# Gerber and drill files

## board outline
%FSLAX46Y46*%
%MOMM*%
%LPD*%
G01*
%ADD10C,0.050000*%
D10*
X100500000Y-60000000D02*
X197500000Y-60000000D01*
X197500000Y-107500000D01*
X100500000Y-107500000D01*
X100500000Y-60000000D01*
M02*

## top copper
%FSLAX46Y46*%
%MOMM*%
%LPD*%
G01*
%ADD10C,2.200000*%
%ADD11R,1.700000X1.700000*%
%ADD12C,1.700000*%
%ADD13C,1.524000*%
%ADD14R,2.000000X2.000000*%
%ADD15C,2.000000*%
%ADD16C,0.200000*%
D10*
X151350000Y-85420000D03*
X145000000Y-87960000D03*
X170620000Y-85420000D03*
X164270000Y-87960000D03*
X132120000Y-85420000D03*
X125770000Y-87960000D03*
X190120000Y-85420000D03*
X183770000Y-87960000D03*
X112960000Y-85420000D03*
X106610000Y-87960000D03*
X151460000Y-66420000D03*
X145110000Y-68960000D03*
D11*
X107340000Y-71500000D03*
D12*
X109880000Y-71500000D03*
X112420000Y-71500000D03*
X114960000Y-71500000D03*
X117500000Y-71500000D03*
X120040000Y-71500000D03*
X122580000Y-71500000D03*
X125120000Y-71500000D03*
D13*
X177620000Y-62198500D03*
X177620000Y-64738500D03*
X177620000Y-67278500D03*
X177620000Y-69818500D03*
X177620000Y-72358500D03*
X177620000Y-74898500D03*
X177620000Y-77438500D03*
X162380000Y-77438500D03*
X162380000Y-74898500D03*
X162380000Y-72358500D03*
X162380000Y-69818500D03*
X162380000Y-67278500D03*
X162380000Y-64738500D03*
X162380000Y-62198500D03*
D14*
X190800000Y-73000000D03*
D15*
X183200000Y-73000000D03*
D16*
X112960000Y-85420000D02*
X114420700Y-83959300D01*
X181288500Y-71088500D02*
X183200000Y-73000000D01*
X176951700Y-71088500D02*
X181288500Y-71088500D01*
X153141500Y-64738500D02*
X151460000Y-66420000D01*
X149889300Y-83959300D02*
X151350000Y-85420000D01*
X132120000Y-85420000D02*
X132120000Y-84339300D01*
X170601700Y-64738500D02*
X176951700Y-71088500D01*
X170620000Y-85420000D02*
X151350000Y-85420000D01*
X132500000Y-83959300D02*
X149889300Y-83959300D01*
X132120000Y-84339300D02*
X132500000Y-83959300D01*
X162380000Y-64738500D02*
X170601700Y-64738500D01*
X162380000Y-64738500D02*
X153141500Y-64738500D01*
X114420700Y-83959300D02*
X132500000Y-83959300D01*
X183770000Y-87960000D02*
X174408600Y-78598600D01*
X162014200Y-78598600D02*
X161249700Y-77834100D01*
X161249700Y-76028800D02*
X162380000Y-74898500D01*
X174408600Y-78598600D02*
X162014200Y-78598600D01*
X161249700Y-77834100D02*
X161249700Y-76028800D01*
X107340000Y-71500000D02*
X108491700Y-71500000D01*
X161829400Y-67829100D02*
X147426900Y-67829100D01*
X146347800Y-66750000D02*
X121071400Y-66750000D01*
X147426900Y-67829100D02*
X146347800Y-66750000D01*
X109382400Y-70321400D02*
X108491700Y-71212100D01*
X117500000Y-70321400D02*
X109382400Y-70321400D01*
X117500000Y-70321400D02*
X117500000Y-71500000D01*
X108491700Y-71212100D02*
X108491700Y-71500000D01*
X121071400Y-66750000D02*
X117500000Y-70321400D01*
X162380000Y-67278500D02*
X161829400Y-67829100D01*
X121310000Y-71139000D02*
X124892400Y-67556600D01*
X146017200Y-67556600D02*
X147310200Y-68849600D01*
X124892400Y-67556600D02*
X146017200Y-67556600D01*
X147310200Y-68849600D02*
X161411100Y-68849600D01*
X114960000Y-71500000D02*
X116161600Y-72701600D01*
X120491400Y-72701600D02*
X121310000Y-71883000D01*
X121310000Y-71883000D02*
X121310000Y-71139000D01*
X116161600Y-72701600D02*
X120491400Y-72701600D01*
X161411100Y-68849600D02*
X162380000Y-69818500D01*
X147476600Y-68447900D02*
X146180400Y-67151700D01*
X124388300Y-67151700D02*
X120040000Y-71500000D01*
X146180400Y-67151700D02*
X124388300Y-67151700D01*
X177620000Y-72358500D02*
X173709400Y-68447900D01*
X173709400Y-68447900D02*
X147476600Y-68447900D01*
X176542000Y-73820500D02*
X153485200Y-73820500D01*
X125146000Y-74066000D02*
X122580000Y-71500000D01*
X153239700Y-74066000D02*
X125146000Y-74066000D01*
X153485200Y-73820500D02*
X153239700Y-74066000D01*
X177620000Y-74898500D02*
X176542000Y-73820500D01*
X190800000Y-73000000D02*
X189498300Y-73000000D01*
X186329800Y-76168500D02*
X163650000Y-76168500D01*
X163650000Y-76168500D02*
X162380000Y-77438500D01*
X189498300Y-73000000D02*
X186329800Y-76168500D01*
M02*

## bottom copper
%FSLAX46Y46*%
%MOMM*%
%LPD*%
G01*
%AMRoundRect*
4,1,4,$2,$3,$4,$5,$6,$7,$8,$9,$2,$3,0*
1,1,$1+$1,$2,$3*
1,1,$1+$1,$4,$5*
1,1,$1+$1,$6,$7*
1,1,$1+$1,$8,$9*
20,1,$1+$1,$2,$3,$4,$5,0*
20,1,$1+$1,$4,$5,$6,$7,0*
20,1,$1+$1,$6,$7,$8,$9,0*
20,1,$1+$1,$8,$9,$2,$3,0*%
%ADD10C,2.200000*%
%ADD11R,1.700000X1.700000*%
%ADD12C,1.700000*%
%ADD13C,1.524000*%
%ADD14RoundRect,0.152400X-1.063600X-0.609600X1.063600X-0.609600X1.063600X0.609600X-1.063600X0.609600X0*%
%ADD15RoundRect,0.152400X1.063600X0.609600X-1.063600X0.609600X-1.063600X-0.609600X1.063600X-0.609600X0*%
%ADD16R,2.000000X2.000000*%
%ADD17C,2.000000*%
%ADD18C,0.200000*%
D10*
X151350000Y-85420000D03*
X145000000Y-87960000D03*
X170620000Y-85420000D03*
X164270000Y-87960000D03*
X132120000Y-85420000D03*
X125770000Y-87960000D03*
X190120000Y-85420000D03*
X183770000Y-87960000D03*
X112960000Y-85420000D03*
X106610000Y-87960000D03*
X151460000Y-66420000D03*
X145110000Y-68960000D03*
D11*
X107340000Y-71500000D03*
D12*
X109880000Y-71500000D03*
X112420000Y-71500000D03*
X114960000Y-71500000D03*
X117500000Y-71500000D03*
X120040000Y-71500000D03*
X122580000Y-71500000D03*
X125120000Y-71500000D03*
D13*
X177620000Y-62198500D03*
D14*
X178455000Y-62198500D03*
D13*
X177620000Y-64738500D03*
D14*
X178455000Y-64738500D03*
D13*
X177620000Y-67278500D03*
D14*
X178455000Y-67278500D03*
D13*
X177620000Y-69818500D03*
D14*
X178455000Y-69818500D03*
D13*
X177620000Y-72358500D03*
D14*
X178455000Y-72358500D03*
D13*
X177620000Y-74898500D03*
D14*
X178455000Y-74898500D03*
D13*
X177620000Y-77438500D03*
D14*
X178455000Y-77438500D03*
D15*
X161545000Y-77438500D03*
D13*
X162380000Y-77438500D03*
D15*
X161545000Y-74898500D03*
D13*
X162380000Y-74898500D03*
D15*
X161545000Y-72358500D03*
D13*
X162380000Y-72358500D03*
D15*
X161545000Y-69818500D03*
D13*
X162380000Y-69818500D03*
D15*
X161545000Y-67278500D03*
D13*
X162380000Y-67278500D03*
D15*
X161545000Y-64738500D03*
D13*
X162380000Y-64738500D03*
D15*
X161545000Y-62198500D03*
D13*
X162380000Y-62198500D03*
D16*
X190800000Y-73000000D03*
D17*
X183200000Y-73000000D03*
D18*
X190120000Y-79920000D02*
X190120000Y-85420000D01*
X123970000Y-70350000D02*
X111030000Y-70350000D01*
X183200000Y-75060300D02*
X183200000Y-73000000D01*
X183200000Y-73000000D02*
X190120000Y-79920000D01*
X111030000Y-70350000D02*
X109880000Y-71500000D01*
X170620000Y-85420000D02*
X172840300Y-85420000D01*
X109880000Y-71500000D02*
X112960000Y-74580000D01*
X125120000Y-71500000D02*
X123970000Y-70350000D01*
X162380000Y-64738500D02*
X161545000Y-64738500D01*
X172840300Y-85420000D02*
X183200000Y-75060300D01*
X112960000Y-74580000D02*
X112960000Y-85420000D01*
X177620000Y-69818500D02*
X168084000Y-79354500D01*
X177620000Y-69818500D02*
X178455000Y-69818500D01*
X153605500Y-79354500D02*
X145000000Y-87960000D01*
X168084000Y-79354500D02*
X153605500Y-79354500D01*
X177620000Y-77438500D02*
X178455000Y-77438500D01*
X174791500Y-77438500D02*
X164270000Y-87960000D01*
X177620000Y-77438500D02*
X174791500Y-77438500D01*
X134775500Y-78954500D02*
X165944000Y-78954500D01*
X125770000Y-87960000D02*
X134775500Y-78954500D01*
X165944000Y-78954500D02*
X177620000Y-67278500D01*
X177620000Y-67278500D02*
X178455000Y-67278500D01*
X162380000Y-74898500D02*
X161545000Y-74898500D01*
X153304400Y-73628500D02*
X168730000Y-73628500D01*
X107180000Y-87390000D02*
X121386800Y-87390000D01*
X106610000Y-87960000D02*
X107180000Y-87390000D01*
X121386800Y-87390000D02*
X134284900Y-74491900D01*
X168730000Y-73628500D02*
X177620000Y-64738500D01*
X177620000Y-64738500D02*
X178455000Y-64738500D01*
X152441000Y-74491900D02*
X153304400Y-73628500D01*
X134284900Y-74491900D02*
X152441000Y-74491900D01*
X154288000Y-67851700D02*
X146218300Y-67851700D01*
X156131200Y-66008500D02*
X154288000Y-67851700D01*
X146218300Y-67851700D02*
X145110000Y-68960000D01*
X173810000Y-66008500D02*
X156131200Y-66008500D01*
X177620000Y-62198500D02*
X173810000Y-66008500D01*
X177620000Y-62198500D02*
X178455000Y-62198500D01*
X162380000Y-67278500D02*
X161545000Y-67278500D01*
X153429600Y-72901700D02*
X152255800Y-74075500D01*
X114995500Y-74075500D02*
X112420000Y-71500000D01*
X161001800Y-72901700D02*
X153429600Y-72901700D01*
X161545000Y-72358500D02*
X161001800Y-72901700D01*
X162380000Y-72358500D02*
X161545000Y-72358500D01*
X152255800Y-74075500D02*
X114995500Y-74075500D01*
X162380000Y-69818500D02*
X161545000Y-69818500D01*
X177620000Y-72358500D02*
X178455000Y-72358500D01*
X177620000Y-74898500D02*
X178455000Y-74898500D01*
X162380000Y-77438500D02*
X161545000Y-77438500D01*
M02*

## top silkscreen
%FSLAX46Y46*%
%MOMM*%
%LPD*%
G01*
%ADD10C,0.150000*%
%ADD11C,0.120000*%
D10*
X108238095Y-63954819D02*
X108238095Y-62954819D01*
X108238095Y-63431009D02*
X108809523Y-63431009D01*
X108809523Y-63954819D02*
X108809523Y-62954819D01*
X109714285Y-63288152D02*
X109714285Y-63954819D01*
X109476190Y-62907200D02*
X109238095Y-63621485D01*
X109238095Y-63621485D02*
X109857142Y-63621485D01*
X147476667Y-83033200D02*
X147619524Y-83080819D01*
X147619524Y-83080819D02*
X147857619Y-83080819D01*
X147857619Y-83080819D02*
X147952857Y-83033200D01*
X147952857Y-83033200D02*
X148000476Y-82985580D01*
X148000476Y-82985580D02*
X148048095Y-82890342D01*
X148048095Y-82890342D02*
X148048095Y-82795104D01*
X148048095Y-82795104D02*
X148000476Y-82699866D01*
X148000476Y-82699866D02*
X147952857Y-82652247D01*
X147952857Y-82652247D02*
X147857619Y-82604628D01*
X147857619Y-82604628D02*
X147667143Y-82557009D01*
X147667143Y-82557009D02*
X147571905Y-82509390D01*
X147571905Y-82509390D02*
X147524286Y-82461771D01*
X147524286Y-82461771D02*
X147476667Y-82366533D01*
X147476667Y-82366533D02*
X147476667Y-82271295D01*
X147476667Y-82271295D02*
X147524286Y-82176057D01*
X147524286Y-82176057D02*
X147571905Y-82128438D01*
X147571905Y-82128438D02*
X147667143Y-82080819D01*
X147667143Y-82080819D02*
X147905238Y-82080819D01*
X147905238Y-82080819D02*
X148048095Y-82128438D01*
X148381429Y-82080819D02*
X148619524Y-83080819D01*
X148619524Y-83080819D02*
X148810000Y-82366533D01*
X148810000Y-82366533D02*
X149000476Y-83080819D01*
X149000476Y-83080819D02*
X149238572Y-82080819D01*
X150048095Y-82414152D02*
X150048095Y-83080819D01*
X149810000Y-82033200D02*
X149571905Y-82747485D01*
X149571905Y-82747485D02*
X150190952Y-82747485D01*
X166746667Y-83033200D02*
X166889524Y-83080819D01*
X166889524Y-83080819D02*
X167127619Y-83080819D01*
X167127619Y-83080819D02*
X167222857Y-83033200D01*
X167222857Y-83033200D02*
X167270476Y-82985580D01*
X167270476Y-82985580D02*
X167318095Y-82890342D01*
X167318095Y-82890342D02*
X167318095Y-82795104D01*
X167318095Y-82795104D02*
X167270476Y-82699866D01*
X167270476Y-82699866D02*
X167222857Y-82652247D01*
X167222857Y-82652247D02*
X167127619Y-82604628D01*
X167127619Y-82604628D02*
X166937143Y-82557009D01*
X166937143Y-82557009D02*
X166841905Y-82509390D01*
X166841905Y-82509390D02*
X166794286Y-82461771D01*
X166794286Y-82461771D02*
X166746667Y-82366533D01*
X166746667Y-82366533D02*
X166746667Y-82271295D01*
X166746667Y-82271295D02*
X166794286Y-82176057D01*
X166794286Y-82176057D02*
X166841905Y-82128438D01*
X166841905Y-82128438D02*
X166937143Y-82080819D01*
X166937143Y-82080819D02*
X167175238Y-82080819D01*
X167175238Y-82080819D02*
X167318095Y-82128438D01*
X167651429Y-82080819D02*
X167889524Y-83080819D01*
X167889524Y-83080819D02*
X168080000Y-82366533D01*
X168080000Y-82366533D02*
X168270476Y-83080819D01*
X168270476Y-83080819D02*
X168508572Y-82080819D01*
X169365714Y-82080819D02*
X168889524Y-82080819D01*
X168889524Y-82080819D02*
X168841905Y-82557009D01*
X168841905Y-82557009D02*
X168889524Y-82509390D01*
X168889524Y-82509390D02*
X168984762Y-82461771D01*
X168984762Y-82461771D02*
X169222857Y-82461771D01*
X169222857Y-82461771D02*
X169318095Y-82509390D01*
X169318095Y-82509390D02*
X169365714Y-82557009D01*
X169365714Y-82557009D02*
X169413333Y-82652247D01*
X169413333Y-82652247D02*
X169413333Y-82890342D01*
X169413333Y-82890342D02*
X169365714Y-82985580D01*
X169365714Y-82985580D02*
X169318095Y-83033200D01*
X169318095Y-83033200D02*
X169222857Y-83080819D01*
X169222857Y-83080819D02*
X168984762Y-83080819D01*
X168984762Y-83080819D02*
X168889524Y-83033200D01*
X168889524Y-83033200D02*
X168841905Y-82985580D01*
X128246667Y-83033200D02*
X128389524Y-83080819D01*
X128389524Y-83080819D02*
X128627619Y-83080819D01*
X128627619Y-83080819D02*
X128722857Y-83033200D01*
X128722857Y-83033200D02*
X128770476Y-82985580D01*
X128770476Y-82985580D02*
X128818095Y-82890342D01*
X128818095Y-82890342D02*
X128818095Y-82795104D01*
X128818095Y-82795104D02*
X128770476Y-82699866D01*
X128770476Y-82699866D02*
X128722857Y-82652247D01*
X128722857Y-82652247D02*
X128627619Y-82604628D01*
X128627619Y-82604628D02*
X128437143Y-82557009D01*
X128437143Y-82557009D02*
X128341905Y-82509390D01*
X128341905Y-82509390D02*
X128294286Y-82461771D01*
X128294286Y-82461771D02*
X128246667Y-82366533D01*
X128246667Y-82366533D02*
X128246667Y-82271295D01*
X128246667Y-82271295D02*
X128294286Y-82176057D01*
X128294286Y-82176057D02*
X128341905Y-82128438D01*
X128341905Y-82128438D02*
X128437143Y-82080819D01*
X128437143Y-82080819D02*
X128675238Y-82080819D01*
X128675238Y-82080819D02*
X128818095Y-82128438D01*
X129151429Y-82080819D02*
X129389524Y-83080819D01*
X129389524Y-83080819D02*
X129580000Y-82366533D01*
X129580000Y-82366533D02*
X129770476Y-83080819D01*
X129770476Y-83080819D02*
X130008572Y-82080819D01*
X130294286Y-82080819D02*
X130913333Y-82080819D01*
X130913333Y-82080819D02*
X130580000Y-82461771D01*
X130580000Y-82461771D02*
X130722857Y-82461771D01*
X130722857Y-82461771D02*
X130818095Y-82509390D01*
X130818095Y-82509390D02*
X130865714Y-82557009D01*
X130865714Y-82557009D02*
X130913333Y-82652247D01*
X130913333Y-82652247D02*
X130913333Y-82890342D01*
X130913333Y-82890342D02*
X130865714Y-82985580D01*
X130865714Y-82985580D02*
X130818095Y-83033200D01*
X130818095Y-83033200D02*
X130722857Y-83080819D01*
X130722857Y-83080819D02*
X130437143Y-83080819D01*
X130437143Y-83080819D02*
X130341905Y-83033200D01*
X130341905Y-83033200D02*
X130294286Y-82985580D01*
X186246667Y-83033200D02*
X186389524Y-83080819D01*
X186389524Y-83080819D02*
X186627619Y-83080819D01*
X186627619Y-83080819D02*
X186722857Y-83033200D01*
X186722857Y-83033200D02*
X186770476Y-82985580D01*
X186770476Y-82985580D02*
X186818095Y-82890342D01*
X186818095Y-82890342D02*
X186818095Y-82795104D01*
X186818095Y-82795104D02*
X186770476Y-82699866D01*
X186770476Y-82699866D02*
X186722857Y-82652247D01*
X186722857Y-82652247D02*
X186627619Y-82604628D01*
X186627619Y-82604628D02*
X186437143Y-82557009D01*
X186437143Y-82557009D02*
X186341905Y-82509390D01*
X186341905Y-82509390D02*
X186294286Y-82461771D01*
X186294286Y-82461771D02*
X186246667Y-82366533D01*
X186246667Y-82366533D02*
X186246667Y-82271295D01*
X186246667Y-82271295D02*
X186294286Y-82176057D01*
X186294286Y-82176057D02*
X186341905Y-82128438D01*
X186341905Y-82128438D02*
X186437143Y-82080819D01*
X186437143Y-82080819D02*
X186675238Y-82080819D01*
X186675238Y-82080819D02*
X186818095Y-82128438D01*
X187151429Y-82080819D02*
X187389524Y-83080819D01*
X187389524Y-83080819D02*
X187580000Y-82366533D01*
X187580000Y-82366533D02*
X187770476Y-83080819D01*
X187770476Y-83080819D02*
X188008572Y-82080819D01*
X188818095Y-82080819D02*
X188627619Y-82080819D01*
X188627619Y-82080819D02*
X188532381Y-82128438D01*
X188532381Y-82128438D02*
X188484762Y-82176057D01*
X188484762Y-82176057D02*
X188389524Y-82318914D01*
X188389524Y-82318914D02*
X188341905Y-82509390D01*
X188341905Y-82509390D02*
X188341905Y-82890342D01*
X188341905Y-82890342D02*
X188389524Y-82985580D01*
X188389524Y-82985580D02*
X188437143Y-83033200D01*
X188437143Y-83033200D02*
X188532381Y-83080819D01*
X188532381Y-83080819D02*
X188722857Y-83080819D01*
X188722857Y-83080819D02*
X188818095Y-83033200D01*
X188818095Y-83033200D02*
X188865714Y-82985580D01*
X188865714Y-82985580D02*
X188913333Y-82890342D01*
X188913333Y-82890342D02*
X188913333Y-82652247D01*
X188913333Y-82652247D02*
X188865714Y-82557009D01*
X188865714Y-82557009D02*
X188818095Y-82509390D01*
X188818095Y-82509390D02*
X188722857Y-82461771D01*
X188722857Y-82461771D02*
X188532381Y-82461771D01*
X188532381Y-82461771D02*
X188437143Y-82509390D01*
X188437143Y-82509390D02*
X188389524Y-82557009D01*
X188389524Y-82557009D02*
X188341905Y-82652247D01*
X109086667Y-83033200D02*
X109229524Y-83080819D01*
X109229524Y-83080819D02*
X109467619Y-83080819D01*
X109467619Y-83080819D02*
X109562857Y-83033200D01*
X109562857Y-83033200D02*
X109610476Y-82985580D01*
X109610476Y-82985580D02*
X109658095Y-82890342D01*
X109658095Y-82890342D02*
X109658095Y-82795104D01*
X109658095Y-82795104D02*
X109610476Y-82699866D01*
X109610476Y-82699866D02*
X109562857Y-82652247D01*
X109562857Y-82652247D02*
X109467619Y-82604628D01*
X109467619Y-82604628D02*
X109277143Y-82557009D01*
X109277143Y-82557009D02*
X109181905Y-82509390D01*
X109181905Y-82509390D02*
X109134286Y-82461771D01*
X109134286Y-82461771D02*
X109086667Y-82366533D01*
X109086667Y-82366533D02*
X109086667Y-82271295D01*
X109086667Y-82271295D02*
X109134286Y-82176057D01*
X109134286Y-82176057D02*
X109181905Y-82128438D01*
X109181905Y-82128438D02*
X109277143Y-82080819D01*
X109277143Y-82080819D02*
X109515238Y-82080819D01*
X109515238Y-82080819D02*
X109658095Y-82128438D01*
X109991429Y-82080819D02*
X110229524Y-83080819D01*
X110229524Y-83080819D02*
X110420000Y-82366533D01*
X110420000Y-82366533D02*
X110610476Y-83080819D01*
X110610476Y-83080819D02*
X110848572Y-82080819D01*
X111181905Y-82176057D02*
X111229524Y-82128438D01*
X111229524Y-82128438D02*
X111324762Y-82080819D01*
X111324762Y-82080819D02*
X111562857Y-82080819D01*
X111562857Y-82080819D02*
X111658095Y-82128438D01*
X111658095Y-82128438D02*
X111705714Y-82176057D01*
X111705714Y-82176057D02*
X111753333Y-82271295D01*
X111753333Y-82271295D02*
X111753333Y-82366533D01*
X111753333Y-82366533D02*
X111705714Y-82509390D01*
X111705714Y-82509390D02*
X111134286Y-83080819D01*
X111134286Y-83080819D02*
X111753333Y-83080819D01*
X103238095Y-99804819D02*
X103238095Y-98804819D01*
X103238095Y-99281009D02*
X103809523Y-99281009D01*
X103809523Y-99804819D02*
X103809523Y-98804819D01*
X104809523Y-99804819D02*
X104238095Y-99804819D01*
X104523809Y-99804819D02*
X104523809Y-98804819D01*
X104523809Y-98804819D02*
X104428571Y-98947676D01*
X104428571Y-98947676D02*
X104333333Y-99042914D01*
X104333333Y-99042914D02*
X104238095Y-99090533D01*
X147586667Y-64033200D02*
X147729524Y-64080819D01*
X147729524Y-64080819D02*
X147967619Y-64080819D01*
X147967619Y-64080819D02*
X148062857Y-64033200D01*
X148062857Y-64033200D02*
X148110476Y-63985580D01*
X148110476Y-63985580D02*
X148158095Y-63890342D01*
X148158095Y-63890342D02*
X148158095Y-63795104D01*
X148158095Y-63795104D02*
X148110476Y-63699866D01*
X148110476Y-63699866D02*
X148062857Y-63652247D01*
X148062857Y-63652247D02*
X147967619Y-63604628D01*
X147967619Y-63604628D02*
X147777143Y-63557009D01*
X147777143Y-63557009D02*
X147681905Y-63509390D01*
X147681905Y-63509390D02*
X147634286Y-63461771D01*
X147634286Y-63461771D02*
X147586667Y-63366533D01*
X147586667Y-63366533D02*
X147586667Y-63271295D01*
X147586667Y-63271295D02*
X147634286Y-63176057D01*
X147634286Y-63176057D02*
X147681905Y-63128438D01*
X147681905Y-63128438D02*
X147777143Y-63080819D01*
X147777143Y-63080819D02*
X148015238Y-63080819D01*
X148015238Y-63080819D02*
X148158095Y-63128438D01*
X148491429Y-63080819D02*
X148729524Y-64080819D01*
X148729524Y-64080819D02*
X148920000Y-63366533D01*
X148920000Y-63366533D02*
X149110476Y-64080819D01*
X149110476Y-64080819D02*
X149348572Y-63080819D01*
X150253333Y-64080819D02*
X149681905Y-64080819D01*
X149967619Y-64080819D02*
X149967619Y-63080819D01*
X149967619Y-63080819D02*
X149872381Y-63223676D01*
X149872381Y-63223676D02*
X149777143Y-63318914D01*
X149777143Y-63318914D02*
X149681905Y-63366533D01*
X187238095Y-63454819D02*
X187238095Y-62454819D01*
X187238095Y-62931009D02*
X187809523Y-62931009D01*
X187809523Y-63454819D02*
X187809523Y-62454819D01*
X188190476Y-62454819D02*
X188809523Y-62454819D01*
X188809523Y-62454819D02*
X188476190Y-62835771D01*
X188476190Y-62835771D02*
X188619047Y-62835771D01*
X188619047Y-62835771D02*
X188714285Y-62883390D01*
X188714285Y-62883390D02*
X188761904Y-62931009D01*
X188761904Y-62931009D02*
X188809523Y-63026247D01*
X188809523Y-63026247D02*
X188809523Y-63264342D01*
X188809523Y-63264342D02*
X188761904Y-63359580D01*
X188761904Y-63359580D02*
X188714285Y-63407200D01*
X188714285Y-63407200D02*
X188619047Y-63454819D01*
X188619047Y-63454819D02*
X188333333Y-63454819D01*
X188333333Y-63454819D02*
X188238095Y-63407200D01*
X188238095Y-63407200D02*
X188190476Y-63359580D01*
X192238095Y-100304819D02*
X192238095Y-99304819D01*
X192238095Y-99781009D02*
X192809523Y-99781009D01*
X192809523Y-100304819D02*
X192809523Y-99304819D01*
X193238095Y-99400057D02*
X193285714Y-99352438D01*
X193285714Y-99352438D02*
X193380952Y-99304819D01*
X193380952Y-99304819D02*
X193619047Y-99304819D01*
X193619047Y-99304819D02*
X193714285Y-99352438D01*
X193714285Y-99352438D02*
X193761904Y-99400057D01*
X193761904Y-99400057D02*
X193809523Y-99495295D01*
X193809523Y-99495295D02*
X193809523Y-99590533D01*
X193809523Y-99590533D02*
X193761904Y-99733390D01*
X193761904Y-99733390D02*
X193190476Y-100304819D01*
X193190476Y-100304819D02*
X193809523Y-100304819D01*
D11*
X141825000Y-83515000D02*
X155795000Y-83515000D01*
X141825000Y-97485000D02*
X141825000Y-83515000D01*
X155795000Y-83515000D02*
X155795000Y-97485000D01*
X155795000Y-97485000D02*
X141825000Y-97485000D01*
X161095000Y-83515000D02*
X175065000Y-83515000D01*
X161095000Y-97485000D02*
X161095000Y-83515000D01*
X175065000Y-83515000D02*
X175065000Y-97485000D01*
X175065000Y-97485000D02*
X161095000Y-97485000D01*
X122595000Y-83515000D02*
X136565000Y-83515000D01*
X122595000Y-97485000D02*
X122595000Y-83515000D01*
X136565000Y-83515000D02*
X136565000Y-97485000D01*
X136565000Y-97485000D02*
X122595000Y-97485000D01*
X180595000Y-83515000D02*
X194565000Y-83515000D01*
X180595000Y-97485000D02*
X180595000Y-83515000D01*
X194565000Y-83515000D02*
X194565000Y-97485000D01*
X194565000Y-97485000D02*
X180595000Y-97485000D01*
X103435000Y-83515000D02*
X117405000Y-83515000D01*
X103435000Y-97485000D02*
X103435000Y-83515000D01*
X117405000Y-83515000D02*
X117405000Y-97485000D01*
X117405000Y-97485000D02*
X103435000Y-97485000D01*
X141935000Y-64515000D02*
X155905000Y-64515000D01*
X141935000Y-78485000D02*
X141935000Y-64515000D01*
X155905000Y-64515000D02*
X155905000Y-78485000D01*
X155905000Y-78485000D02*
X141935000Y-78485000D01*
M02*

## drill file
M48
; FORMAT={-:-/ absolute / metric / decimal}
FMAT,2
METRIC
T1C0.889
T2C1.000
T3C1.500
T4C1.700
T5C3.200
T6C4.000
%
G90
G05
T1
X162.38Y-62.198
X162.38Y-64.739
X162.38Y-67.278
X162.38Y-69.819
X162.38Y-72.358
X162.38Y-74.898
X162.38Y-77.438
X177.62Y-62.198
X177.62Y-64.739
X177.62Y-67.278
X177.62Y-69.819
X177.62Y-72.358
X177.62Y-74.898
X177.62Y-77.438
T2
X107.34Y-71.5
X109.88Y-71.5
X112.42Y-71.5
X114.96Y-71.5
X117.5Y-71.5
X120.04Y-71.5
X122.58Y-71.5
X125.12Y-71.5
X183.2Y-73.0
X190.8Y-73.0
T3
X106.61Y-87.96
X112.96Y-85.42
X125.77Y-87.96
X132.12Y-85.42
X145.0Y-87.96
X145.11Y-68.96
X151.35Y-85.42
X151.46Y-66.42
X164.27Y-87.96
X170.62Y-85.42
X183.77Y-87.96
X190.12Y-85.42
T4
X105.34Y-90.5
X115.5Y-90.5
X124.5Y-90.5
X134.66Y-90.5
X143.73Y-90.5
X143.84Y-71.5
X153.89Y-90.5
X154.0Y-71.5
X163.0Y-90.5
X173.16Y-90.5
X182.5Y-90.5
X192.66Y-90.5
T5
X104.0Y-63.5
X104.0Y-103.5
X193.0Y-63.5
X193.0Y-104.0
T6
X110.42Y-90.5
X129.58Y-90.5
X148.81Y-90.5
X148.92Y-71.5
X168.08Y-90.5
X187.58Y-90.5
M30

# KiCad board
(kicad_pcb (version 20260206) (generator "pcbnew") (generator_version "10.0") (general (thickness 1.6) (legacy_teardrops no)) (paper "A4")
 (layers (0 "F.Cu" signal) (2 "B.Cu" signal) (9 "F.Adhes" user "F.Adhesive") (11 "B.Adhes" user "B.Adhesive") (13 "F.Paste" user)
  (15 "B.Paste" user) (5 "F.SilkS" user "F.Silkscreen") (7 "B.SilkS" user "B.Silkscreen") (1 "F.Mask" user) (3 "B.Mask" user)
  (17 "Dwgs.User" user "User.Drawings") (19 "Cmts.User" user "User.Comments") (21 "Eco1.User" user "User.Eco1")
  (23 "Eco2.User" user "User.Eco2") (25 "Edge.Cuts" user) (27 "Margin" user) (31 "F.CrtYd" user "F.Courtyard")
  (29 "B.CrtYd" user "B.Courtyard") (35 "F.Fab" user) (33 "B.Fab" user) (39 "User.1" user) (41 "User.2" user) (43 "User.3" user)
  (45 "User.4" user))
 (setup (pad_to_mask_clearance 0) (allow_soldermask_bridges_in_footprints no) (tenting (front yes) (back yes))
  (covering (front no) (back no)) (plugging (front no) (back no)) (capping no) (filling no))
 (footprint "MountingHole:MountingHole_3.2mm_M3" (layer "F.Cu") (at 104 63.5)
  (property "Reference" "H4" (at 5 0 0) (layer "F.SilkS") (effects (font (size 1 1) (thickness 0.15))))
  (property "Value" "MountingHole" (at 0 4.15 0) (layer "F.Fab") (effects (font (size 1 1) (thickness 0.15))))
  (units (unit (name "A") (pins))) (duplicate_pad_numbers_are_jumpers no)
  (pad "" np_thru_hole circle (at 0 0) (size 3.2 3.2) (drill 3.2) (layers "*.Cu" "*.Mask")))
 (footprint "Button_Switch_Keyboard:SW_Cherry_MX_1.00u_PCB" (layer "F.Cu") (at 151.35 85.42)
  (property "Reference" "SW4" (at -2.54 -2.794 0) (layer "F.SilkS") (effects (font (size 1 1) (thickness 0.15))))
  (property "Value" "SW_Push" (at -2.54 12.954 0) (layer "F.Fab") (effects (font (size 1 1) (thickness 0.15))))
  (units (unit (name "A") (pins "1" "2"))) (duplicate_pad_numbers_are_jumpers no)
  (fp_line (start -9.525 -1.905) (end 4.445 -1.905) (stroke (width 0.12) (type solid)) (layer "F.SilkS"))
  (fp_line (start -9.525 12.065) (end -9.525 -1.905) (stroke (width 0.12) (type solid)) (layer "F.SilkS"))
  (fp_line (start 4.445 -1.905) (end 4.445 12.065) (stroke (width 0.12) (type solid)) (layer "F.SilkS"))
  (fp_line (start 4.445 12.065) (end -9.525 12.065) (stroke (width 0.12) (type solid)) (layer "F.SilkS"))
  (pad "" np_thru_hole circle (at -7.62 5.08) (size 1.7 1.7) (drill 1.7) (layers "*.Cu" "*.Mask"))
  (pad "" np_thru_hole circle (at -2.54 5.08) (size 4 4) (drill 4) (layers "*.Cu" "*.Mask"))
  (pad "" np_thru_hole circle (at 2.54 5.08) (size 1.7 1.7) (drill 1.7) (layers "*.Cu" "*.Mask"))
  (pad "1" thru_hole circle (at 0 0) (size 2.2 2.2) (drill 1.5) (layers "*.Cu" "*.Mask") (remove_unused_layers no) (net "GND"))
  (pad "2" thru_hole circle (at -6.35 2.54) (size 2.2 2.2) (drill 1.5) (layers "*.Cu" "*.Mask") (remove_unused_layers no)
   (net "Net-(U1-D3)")))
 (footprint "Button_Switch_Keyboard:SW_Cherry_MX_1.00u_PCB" (layer "F.Cu") (at 170.62 85.42)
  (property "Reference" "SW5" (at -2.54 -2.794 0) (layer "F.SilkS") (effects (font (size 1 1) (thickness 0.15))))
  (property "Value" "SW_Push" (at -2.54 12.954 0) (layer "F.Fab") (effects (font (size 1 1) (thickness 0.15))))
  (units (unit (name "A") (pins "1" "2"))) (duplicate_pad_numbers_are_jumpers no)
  (fp_line (start -9.525 -1.905) (end 4.445 -1.905) (stroke (width 0.12) (type solid)) (layer "F.SilkS"))
  (fp_line (start -9.525 12.065) (end -9.525 -1.905) (stroke (width 0.12) (type solid)) (layer "F.SilkS"))
  (fp_line (start 4.445 -1.905) (end 4.445 12.065) (stroke (width 0.12) (type solid)) (layer "F.SilkS"))
  (fp_line (start 4.445 12.065) (end -9.525 12.065) (stroke (width 0.12) (type solid)) (layer "F.SilkS"))
  (pad "" np_thru_hole circle (at -7.62 5.08) (size 1.7 1.7) (drill 1.7) (layers "*.Cu" "*.Mask"))
  (pad "" np_thru_hole circle (at -2.54 5.08) (size 4 4) (drill 4) (layers "*.Cu" "*.Mask"))
  (pad "" np_thru_hole circle (at 2.54 5.08) (size 1.7 1.7) (drill 1.7) (layers "*.Cu" "*.Mask"))
  (pad "1" thru_hole circle (at 0 0) (size 2.2 2.2) (drill 1.5) (layers "*.Cu" "*.Mask") (remove_unused_layers no) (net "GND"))
  (pad "2" thru_hole circle (at -6.35 2.54) (size 2.2 2.2) (drill 1.5) (layers "*.Cu" "*.Mask") (remove_unused_layers no)
   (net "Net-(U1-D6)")))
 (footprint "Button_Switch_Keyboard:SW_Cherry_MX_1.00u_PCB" (layer "F.Cu") (at 132.12 85.42)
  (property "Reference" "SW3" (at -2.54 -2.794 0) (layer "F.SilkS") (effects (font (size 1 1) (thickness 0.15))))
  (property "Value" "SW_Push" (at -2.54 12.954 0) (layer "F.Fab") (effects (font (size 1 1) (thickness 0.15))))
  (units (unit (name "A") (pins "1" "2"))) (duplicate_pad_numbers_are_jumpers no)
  (fp_line (start -9.525 -1.905) (end 4.445 -1.905) (stroke (width 0.12) (type solid)) (layer "F.SilkS"))
  (fp_line (start -9.525 12.065) (end -9.525 -1.905) (stroke (width 0.12) (type solid)) (layer "F.SilkS"))
  (fp_line (start 4.445 -1.905) (end 4.445 12.065) (stroke (width 0.12) (type solid)) (layer "F.SilkS"))
  (fp_line (start 4.445 12.065) (end -9.525 12.065) (stroke (width 0.12) (type solid)) (layer "F.SilkS"))
  (pad "" np_thru_hole circle (at -7.62 5.08) (size 1.7 1.7) (drill 1.7) (layers "*.Cu" "*.Mask"))
  (pad "" np_thru_hole circle (at -2.54 5.08) (size 4 4) (drill 4) (layers "*.Cu" "*.Mask"))
  (pad "" np_thru_hole circle (at 2.54 5.08) (size 1.7 1.7) (drill 1.7) (layers "*.Cu" "*.Mask"))
  (pad "1" thru_hole circle (at 0 0) (size 2.2 2.2) (drill 1.5) (layers "*.Cu" "*.Mask") (remove_unused_layers no) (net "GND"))
  (pad "2" thru_hole circle (at -6.35 2.54) (size 2.2 2.2) (drill 1.5) (layers "*.Cu" "*.Mask") (remove_unused_layers no)
   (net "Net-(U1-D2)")))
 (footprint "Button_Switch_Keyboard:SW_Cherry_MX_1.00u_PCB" (layer "F.Cu") (at 190.12 85.42)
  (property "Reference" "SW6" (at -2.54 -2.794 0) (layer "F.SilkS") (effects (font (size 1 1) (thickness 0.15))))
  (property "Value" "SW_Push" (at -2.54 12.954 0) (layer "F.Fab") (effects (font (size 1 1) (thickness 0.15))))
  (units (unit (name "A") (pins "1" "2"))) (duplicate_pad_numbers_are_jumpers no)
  (fp_line (start -9.525 -1.905) (end 4.445 -1.905) (stroke (width 0.12) (type solid)) (layer "F.SilkS"))
  (fp_line (start -9.525 12.065) (end -9.525 -1.905) (stroke (width 0.12) (type solid)) (layer "F.SilkS"))
  (fp_line (start 4.445 -1.905) (end 4.445 12.065) (stroke (width 0.12) (type solid)) (layer "F.SilkS"))
  (fp_line (start 4.445 12.065) (end -9.525 12.065) (stroke (width 0.12) (type solid)) (layer "F.SilkS"))
  (pad "" np_thru_hole circle (at -7.62 5.08) (size 1.7 1.7) (drill 1.7) (layers "*.Cu" "*.Mask"))
  (pad "" np_thru_hole circle (at -2.54 5.08) (size 4 4) (drill 4) (layers "*.Cu" "*.Mask"))
  (pad "" np_thru_hole circle (at 2.54 5.08) (size 1.7 1.7) (drill 1.7) (layers "*.Cu" "*.Mask"))
  (pad "1" thru_hole circle (at 0 0) (size 2.2 2.2) (drill 1.5) (layers "*.Cu" "*.Mask") (remove_unused_layers no) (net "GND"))
  (pad "2" thru_hole circle (at -6.35 2.54) (size 2.2 2.2) (drill 1.5) (layers "*.Cu" "*.Mask") (remove_unused_layers no)
   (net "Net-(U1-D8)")))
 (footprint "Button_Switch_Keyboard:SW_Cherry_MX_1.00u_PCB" (layer "F.Cu") (at 112.96 85.42)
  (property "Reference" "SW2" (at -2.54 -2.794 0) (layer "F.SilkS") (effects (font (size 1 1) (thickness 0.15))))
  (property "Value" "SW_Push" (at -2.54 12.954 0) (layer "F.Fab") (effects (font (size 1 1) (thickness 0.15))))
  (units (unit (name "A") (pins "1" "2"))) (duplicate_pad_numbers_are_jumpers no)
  (fp_line (start -9.525 -1.905) (end 4.445 -1.905) (stroke (width 0.12) (type solid)) (layer "F.SilkS"))
  (fp_line (start -9.525 12.065) (end -9.525 -1.905) (stroke (width 0.12) (type solid)) (layer "F.SilkS"))
  (fp_line (start 4.445 -1.905) (end 4.445 12.065) (stroke (width 0.12) (type solid)) (layer "F.SilkS"))
  (fp_line (start 4.445 12.065) (end -9.525 12.065) (stroke (width 0.12) (type solid)) (layer "F.SilkS"))
  (pad "" np_thru_hole circle (at -7.62 5.08) (size 1.7 1.7) (drill 1.7) (layers "*.Cu" "*.Mask"))
  (pad "" np_thru_hole circle (at -2.54 5.08) (size 4 4) (drill 4) (layers "*.Cu" "*.Mask"))
  (pad "" np_thru_hole circle (at 2.54 5.08) (size 1.7 1.7) (drill 1.7) (layers "*.Cu" "*.Mask"))
  (pad "1" thru_hole circle (at 0 0) (size 2.2 2.2) (drill 1.5) (layers "*.Cu" "*.Mask") (remove_unused_layers no) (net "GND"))
  (pad "2" thru_hole circle (at -6.35 2.54) (size 2.2 2.2) (drill 1.5) (layers "*.Cu" "*.Mask") (remove_unused_layers no)
   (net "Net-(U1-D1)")))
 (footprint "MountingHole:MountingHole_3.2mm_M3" (layer "F.Cu") (at 104 103.5)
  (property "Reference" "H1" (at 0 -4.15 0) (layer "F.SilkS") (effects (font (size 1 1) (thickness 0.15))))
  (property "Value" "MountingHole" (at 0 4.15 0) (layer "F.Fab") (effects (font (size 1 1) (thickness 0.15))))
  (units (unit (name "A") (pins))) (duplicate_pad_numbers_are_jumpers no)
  (pad "" np_thru_hole circle (at 0 0) (size 3.2 3.2) (drill 3.2) (layers "*.Cu" "*.Mask")))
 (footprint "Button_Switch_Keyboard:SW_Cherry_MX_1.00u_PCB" (layer "F.Cu") (at 151.46 66.42)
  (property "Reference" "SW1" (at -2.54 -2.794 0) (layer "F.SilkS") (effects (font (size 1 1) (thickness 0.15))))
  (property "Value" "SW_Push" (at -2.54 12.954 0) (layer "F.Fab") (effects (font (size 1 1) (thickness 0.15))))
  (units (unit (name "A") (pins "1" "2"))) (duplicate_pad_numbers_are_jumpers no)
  (fp_line (start -9.525 -1.905) (end 4.445 -1.905) (stroke (width 0.12) (type solid)) (layer "F.SilkS"))
  (fp_line (start -9.525 12.065) (end -9.525 -1.905) (stroke (width 0.12) (type solid)) (layer "F.SilkS"))
  (fp_line (start 4.445 -1.905) (end 4.445 12.065) (stroke (width 0.12) (type solid)) (layer "F.SilkS"))
  (fp_line (start 4.445 12.065) (end -9.525 12.065) (stroke (width 0.12) (type solid)) (layer "F.SilkS"))
  (pad "" np_thru_hole circle (at -7.62 5.08) (size 1.7 1.7) (drill 1.7) (layers "*.Cu" "*.Mask"))
  (pad "" np_thru_hole circle (at -2.54 5.08) (size 4 4) (drill 4) (layers "*.Cu" "*.Mask"))
  (pad "" np_thru_hole circle (at 2.54 5.08) (size 1.7 1.7) (drill 1.7) (layers "*.Cu" "*.Mask"))
  (pad "1" thru_hole circle (at 0 0) (size 2.2 2.2) (drill 1.5) (layers "*.Cu" "*.Mask") (remove_unused_layers no) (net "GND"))
  (pad "2" thru_hole circle (at -6.35 2.54) (size 2.2 2.2) (drill 1.5) (layers "*.Cu" "*.Mask") (remove_unused_layers no)
   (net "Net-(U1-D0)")))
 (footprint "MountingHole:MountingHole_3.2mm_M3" (layer "F.Cu") (at 193 63.5)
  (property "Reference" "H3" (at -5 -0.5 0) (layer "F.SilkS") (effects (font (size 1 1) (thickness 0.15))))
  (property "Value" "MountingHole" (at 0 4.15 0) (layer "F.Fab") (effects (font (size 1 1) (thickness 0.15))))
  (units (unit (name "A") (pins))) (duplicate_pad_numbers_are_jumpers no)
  (pad "" np_thru_hole circle (at 0 0) (size 3.2 3.2) (drill 3.2) (layers "*.Cu" "*.Mask")))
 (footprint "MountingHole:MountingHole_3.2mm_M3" (layer "F.Cu") (at 193 104)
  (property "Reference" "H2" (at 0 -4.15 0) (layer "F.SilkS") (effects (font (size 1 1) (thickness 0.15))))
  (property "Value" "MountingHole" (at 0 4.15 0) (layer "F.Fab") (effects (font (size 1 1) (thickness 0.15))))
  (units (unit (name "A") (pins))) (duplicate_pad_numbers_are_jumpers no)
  (pad "" np_thru_hole circle (at 0 0) (size 3.2 3.2) (drill 3.2) (layers "*.Cu" "*.Mask")))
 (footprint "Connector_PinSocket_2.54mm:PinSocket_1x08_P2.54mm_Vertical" (layer "B.Cu") (at 107.34 71.5 -90)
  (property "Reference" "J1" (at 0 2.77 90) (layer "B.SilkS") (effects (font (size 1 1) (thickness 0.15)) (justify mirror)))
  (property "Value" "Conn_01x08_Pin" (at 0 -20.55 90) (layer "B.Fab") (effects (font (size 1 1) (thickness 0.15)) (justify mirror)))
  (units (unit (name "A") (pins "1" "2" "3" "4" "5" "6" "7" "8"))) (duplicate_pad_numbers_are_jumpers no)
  (pad "1" thru_hole rect (at 0 0 270) (size 1.7 1.7) (drill 1) (layers "*.Cu" "*.Mask") (remove_unused_layers no) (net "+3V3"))
  (pad "2" thru_hole circle (at 0 -2.54 270) (size 1.7 1.7) (drill 1) (layers "*.Cu" "*.Mask") (remove_unused_layers no) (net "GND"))
  (pad "3" thru_hole circle (at 0 -5.08 270) (size 1.7 1.7) (drill 1) (layers "*.Cu" "*.Mask") (remove_unused_layers no) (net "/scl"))
  (pad "4" thru_hole circle (at 0 -7.62 270) (size 1.7 1.7) (drill 1) (layers "*.Cu" "*.Mask") (remove_unused_layers no) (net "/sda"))
  (pad "5" thru_hole circle (at 0 -10.16 270) (size 1.7 1.7) (drill 1) (layers "*.Cu" "*.Mask") (remove_unused_layers no) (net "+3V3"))
  (pad "6" thru_hole circle (at 0 -12.7 270) (size 1.7 1.7) (drill 1) (layers "*.Cu" "*.Mask") (remove_unused_layers no) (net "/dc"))
  (pad "7" thru_hole circle (at 0 -15.24 270) (size 1.7 1.7) (drill 1) (layers "*.Cu" "*.Mask") (remove_unused_layers no) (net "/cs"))
  (pad "8" thru_hole circle (at 0 -17.78 270) (size 1.7 1.7) (drill 1) (layers "*.Cu" "*.Mask") (remove_unused_layers no) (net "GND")))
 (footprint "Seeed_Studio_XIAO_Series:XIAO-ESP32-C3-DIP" (layer "B.Cu") (at 170 69.8185 90)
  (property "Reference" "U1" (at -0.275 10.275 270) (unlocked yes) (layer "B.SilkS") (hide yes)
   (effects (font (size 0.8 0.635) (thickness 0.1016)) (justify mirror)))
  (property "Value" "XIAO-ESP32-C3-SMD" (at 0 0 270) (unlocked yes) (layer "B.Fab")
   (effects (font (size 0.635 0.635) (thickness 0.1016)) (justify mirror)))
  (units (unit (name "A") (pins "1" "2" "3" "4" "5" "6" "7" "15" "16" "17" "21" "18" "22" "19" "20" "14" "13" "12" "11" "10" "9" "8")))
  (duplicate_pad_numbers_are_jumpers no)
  (pad "1" thru_hole circle (at 7.62 7.62) (size 1.524 1.524) (drill 0.889) (layers "*.Cu" "*.Mask") (remove_unused_layers no)
   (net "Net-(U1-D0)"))
  (pad "1" smd roundrect (at 7.62 8.455) (size 2.432 1.524) (layers "B.Cu" "B.Mask") (roundrect_rratio 0.1) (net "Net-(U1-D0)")
   (thermal_bridge_angle 45))
  (pad "2" thru_hole circle (at 5.08 7.62) (size 1.524 1.524) (drill 0.889) (layers "*.Cu" "*.Mask") (remove_unused_layers no)
   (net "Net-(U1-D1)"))
  (pad "2" smd roundrect (at 5.08 8.455) (size 2.432 1.524) (layers "B.Cu" "B.Mask") (roundrect_rratio 0.1) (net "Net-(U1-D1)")
   (thermal_bridge_angle 45))
  (pad "3" thru_hole circle (at 2.54 7.62) (size 1.524 1.524) (drill 0.889) (layers "*.Cu" "*.Mask") (remove_unused_layers no)
   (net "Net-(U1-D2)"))
  (pad "3" smd roundrect (at 2.54 8.455) (size 2.432 1.524) (layers "B.Cu" "B.Mask") (roundrect_rratio 0.1) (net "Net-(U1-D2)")
   (thermal_bridge_angle 45))
  (pad "4" thru_hole circle (at 0 7.62) (size 1.524 1.524) (drill 0.889) (layers "*.Cu" "*.Mask") (remove_unused_layers no)
   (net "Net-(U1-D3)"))
  (pad "4" smd roundrect (at 0 8.455) (size 2.432 1.524) (layers "B.Cu" "B.Mask") (roundrect_rratio 0.1) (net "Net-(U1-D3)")
   (thermal_bridge_angle 45))
  (pad "5" thru_hole circle (at -2.54 7.62) (size 1.524 1.524) (drill 0.889) (layers "*.Cu" "*.Mask") (remove_unused_layers no) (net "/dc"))
  (pad "5" smd roundrect (at -2.54 8.455) (size 2.432 1.524) (layers "B.Cu" "B.Mask") (roundrect_rratio 0.1) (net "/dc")
   (thermal_bridge_angle 45))
  (pad "6" thru_hole circle (at -5.08 7.62) (size 1.524 1.524) (drill 0.889) (layers "*.Cu" "*.Mask") (remove_unused_layers no) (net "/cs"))
  (pad "6" smd roundrect (at -5.08 8.455) (size 2.432 1.524) (layers "B.Cu" "B.Mask") (roundrect_rratio 0.1) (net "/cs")
   (thermal_bridge_angle 45))
  (pad "7" thru_hole circle (at -7.62 7.62) (size 1.524 1.524) (drill 0.889) (layers "*.Cu" "*.Mask") (remove_unused_layers no)
   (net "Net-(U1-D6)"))
  (pad "7" smd roundrect (at -7.62 8.455) (size 2.432 1.524) (layers "B.Cu" "B.Mask") (roundrect_rratio 0.1) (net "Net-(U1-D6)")
   (thermal_bridge_angle 45))
  (pad "8" smd roundrect (at -7.62 -8.455 180) (size 2.432 1.524) (layers "B.Cu" "B.Mask") (roundrect_rratio 0.1) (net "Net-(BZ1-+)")
   (thermal_bridge_angle 45))
  (pad "8" thru_hole circle (at -7.62 -7.62 180) (size 1.524 1.524) (drill 0.889) (layers "*.Cu" "*.Mask") (remove_unused_layers no)
   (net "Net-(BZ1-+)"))
  (pad "9" smd roundrect (at -5.08 -8.455 180) (size 2.432 1.524) (layers "B.Cu" "B.Mask") (roundrect_rratio 0.1) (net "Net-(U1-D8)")
   (thermal_bridge_angle 45))
  (pad "9" thru_hole circle (at -5.08 -7.62 180) (size 1.524 1.524) (drill 0.889) (layers "*.Cu" "*.Mask") (remove_unused_layers no)
   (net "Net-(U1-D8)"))
  (pad "10" smd roundrect (at -2.54 -8.455 180) (size 2.432 1.524) (layers "B.Cu" "B.Mask") (roundrect_rratio 0.1) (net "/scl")
   (thermal_bridge_angle 45))
  (pad "10" thru_hole circle (at -2.54 -7.62 180) (size 1.524 1.524) (drill 0.889) (layers "*.Cu" "*.Mask") (remove_unused_layers no)
   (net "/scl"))
  (pad "11" smd roundrect (at 0 -8.455 180) (size 2.432 1.524) (layers "B.Cu" "B.Mask") (roundrect_rratio 0.1) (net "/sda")
   (thermal_bridge_angle 45))
  (pad "11" thru_hole circle (at 0 -7.62 180) (size 1.524 1.524) (drill 0.889) (layers "*.Cu" "*.Mask") (remove_unused_layers no)
   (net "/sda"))
  (pad "12" smd roundrect (at 2.54 -8.455 180) (size 2.432 1.524) (layers "B.Cu" "B.Mask") (roundrect_rratio 0.1) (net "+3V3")
   (thermal_bridge_angle 45))
  (pad "12" thru_hole circle (at 2.54 -7.62 180) (size 1.524 1.524) (drill 0.889) (layers "*.Cu" "*.Mask") (remove_unused_layers no)
   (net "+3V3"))
  (pad "13" smd roundrect (at 5.08 -8.455 180) (size 2.432 1.524) (layers "B.Cu" "B.Mask") (roundrect_rratio 0.1) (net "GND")
   (thermal_bridge_angle 45))
  (pad "13" thru_hole circle (at 5.08 -7.62 180) (size 1.524 1.524) (drill 0.889) (layers "*.Cu" "*.Mask") (remove_unused_layers no)
   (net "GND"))
  (pad "14" smd roundrect (at 7.62 -8.455 180) (size 2.432 1.524) (layers "B.Cu" "B.Mask") (roundrect_rratio 0.1)
   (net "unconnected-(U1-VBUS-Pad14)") (thermal_bridge_angle 45))
  (pad "14" thru_hole circle (at 7.62 -7.62 180) (size 1.524 1.524) (drill 0.889) (layers "*.Cu" "*.Mask") (remove_unused_layers no)
   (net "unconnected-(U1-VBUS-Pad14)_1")))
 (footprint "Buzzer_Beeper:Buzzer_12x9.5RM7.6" (layer "B.Cu") (at 190.8 73 180)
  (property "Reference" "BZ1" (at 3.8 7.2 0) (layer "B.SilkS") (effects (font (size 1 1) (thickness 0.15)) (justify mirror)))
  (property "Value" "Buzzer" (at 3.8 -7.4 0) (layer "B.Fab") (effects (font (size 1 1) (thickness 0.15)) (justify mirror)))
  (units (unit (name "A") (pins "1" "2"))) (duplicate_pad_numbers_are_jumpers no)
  (pad "1" thru_hole rect (at 0 0 180) (size 2 2) (drill 1) (layers "*.Cu" "*.Mask") (remove_unused_layers no) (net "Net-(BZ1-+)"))
  (pad "2" thru_hole circle (at 7.6 0 180) (size 2 2) (drill 1) (layers "*.Cu" "*.Mask") (remove_unused_layers no) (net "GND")))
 (gr_rect (start 100.5 60) (end 197.5 107.5) (stroke (width 0.05) (type default)) (fill no) (layer "Edge.Cuts"))
 (segment (start 112.96 85.42) (end 114.4207 83.9593) (width 0.2) (layer "F.Cu") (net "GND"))
 (segment (start 181.2885 71.0885) (end 183.2 73) (width 0.2) (layer "F.Cu") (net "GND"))
 (segment (start 176.9517 71.0885) (end 181.2885 71.0885) (width 0.2) (layer "F.Cu") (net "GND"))
 (segment (start 153.1415 64.7385) (end 151.46 66.42) (width 0.2) (layer "F.Cu") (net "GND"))
 (segment (start 149.8893 83.9593) (end 151.35 85.42) (width 0.2) (layer "F.Cu") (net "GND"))
 (segment (start 132.12 85.42) (end 132.12 84.3393) (width 0.2) (layer "F.Cu") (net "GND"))
 (segment (start 170.6017 64.7385) (end 176.9517 71.0885) (width 0.2) (layer "F.Cu") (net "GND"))
 (segment (start 170.62 85.42) (end 151.35 85.42) (width 0.2) (layer "F.Cu") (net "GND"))
 (segment (start 132.5 83.9593) (end 149.8893 83.9593) (width 0.2) (layer "F.Cu") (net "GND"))
 (segment (start 132.12 84.3393) (end 132.5 83.9593) (width 0.2) (layer "F.Cu") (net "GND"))
 (segment (start 162.38 64.7385) (end 170.6017 64.7385) (width 0.2) (layer "F.Cu") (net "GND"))
 (segment (start 162.38 64.7385) (end 153.1415 64.7385) (width 0.2) (layer "F.Cu") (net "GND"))
 (segment (start 114.4207 83.9593) (end 132.5 83.9593) (width 0.2) (layer "F.Cu") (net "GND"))
 (segment (start 190.12 79.92) (end 190.12 85.42) (width 0.2) (layer "B.Cu") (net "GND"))
 (segment (start 123.97 70.35) (end 111.03 70.35) (width 0.2) (layer "B.Cu") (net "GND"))
 (segment (start 183.2 75.0603) (end 183.2 73) (width 0.2) (layer "B.Cu") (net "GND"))
 (segment (start 183.2 73) (end 190.12 79.92) (width 0.2) (layer "B.Cu") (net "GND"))
 (segment (start 111.03 70.35) (end 109.88 71.5) (width 0.2) (layer "B.Cu") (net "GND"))
 (segment (start 170.62 85.42) (end 172.8403 85.42) (width 0.2) (layer "B.Cu") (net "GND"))
 (segment (start 109.88 71.5) (end 112.96 74.58) (width 0.2) (layer "B.Cu") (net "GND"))
 (segment (start 125.12 71.5) (end 123.97 70.35) (width 0.2) (layer "B.Cu") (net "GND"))
 (segment (start 162.38 64.7385) (end 161.545 64.7385) (width 0.2) (layer "B.Cu") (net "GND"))
 (segment (start 172.8403 85.42) (end 183.2 75.0603) (width 0.2) (layer "B.Cu") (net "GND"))
 (segment (start 112.96 74.58) (end 112.96 85.42) (width 0.2) (layer "B.Cu") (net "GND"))
 (segment (start 177.62 69.8185) (end 168.084 79.3545) (width 0.2) (layer "B.Cu") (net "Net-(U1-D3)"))
 (segment (start 177.62 69.8185) (end 178.455 69.8185) (width 0.2) (layer "B.Cu") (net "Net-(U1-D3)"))
 (segment (start 153.6055 79.3545) (end 145 87.96) (width 0.2) (layer "B.Cu") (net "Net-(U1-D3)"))
 (segment (start 168.084 79.3545) (end 153.6055 79.3545) (width 0.2) (layer "B.Cu") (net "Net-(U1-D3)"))
 (segment (start 177.62 77.4385) (end 178.455 77.4385) (width 0.2) (layer "B.Cu") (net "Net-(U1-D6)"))
 (segment (start 174.7915 77.4385) (end 164.27 87.96) (width 0.2) (layer "B.Cu") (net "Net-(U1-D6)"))
 (segment (start 177.62 77.4385) (end 174.7915 77.4385) (width 0.2) (layer "B.Cu") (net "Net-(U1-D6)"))
 (segment (start 134.7755 78.9545) (end 165.944 78.9545) (width 0.2) (layer "B.Cu") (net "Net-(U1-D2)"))
 (segment (start 125.77 87.96) (end 134.7755 78.9545) (width 0.2) (layer "B.Cu") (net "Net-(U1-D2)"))
 (segment (start 165.944 78.9545) (end 177.62 67.2785) (width 0.2) (layer "B.Cu") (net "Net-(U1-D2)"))
 (segment (start 177.62 67.2785) (end 178.455 67.2785) (width 0.2) (layer "B.Cu") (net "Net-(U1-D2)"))
 (segment (start 183.77 87.96) (end 174.4086 78.5986) (width 0.2) (layer "F.Cu") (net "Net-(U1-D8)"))
 (segment (start 162.0142 78.5986) (end 161.2497 77.8341) (width 0.2) (layer "F.Cu") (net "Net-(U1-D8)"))
 (segment (start 161.2497 76.0288) (end 162.38 74.8985) (width 0.2) (layer "F.Cu") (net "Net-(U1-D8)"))
 (segment (start 174.4086 78.5986) (end 162.0142 78.5986) (width 0.2) (layer "F.Cu") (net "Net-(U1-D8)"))
 (segment (start 161.2497 77.8341) (end 161.2497 76.0288) (width 0.2) (layer "F.Cu") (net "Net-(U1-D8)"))
 (segment (start 162.38 74.8985) (end 161.545 74.8985) (width 0.2) (layer "B.Cu") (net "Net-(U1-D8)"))
 (segment (start 153.3044 73.6285) (end 168.73 73.6285) (width 0.2) (layer "B.Cu") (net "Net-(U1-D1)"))
 (segment (start 107.18 87.39) (end 121.3868 87.39) (width 0.2) (layer "B.Cu") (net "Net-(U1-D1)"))
 (segment (start 106.61 87.96) (end 107.18 87.39) (width 0.2) (layer "B.Cu") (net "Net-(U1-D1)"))
 (segment (start 121.3868 87.39) (end 134.2849 74.4919) (width 0.2) (layer "B.Cu") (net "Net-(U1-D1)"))
 (segment (start 168.73 73.6285) (end 177.62 64.7385) (width 0.2) (layer "B.Cu") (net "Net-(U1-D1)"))
 (segment (start 177.62 64.7385) (end 178.455 64.7385) (width 0.2) (layer "B.Cu") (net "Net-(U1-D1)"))
 (segment (start 152.441 74.4919) (end 153.3044 73.6285) (width 0.2) (layer "B.Cu") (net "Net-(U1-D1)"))
 (segment (start 134.2849 74.4919) (end 152.441 74.4919) (width 0.2) (layer "B.Cu") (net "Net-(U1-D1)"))
 (segment (start 154.288 67.8517) (end 146.2183 67.8517) (width 0.2) (layer "B.Cu") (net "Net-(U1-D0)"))
 (segment (start 156.1312 66.0085) (end 154.288 67.8517) (width 0.2) (layer "B.Cu") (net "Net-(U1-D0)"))
 (segment (start 146.2183 67.8517) (end 145.11 68.96) (width 0.2) (layer "B.Cu") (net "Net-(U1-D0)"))
 (segment (start 173.81 66.0085) (end 156.1312 66.0085) (width 0.2) (layer "B.Cu") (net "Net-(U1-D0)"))
 (segment (start 177.62 62.1985) (end 173.81 66.0085) (width 0.2) (layer "B.Cu") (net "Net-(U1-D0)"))
 (segment (start 177.62 62.1985) (end 178.455 62.1985) (width 0.2) (layer "B.Cu") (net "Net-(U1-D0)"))
 (segment (start 107.34 71.5) (end 108.4917 71.5) (width 0.2) (layer "F.Cu") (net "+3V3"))
 (segment (start 161.8294 67.8291) (end 147.4269 67.8291) (width 0.2) (layer "F.Cu") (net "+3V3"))
 (segment (start 146.3478 66.75) (end 121.0714 66.75) (width 0.2) (layer "F.Cu") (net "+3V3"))
 (segment (start 147.4269 67.8291) (end 146.3478 66.75) (width 0.2) (layer "F.Cu") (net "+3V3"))
 (segment (start 109.3824 70.3214) (end 108.4917 71.2121) (width 0.2) (layer "F.Cu") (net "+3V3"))
 (segment (start 117.5 70.3214) (end 109.3824 70.3214) (width 0.2) (layer "F.Cu") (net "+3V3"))
 (segment (start 117.5 70.3214) (end 117.5 71.5) (width 0.2) (layer "F.Cu") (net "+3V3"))
 (segment (start 108.4917 71.2121) (end 108.4917 71.5) (width 0.2) (layer "F.Cu") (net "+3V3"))
 (segment (start 121.0714 66.75) (end 117.5 70.3214) (width 0.2) (layer "F.Cu") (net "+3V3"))
 (segment (start 162.38 67.2785) (end 161.8294 67.8291) (width 0.2) (layer "F.Cu") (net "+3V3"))
 (segment (start 162.38 67.2785) (end 161.545 67.2785) (width 0.2) (layer "B.Cu") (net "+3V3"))
 (segment (start 153.4296 72.9017) (end 152.2558 74.0755) (width 0.2) (layer "B.Cu") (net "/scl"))
 (segment (start 114.9955 74.0755) (end 112.42 71.5) (width 0.2) (layer "B.Cu") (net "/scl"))
 (segment (start 161.0018 72.9017) (end 153.4296 72.9017) (width 0.2) (layer "B.Cu") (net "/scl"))
 (segment (start 161.545 72.3585) (end 161.0018 72.9017) (width 0.2) (layer "B.Cu") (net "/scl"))
 (segment (start 162.38 72.3585) (end 161.545 72.3585) (width 0.2) (layer "B.Cu") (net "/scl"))
 (segment (start 152.2558 74.0755) (end 114.9955 74.0755) (width 0.2) (layer "B.Cu") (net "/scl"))
 (segment (start 121.31 71.139) (end 124.8924 67.5566) (width 0.2) (layer "F.Cu") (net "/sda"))
 (segment (start 146.0172 67.5566) (end 147.3102 68.8496) (width 0.2) (layer "F.Cu") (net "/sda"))
 (segment (start 124.8924 67.5566) (end 146.0172 67.5566) (width 0.2) (layer "F.Cu") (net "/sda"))
 (segment (start 147.3102 68.8496) (end 161.4111 68.8496) (width 0.2) (layer "F.Cu") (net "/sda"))
 (segment (start 114.96 71.5) (end 116.1616 72.7016) (width 0.2) (layer "F.Cu") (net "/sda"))
 (segment (start 120.4914 72.7016) (end 121.31 71.883) (width 0.2) (layer "F.Cu") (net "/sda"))
 (segment (start 121.31 71.883) (end 121.31 71.139) (width 0.2) (layer "F.Cu") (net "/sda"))
 (segment (start 116.1616 72.7016) (end 120.4914 72.7016) (width 0.2) (layer "F.Cu") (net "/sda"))
 (segment (start 161.4111 68.8496) (end 162.38 69.8185) (width 0.2) (layer "F.Cu") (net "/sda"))
 (segment (start 162.38 69.8185) (end 161.545 69.8185) (width 0.2) (layer "B.Cu") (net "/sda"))
 (segment (start 147.4766 68.4479) (end 146.1804 67.1517) (width 0.2) (layer "F.Cu") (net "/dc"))
 (segment (start 124.3883 67.1517) (end 120.04 71.5) (width 0.2) (layer "F.Cu") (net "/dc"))
 (segment (start 146.1804 67.1517) (end 124.3883 67.1517) (width 0.2) (layer "F.Cu") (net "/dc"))
 (segment (start 177.62 72.3585) (end 173.7094 68.4479) (width 0.2) (layer "F.Cu") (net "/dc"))
 (segment (start 173.7094 68.4479) (end 147.4766 68.4479) (width 0.2) (layer "F.Cu") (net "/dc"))
 (segment (start 177.62 72.3585) (end 178.455 72.3585) (width 0.2) (layer "B.Cu") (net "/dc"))
 (segment (start 176.542 73.8205) (end 153.4852 73.8205) (width 0.2) (layer "F.Cu") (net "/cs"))
 (segment (start 125.146 74.066) (end 122.58 71.5) (width 0.2) (layer "F.Cu") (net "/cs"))
 (segment (start 153.2397 74.066) (end 125.146 74.066) (width 0.2) (layer "F.Cu") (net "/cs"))
 (segment (start 153.4852 73.8205) (end 153.2397 74.066) (width 0.2) (layer "F.Cu") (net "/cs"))
 (segment (start 177.62 74.8985) (end 176.542 73.8205) (width 0.2) (layer "F.Cu") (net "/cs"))
 (segment (start 177.62 74.8985) (end 178.455 74.8985) (width 0.2) (layer "B.Cu") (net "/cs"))
 (segment (start 190.8 73) (end 189.4983 73) (width 0.2) (layer "F.Cu") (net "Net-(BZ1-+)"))
 (segment (start 186.3298 76.1685) (end 163.65 76.1685) (width 0.2) (layer "F.Cu") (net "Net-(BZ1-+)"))
 (segment (start 163.65 76.1685) (end 162.38 77.4385) (width 0.2) (layer "F.Cu") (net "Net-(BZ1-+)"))
 (segment (start 189.4983 73) (end 186.3298 76.1685) (width 0.2) (layer "F.Cu") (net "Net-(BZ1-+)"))
 (segment (start 162.38 77.4385) (end 161.545 77.4385) (width 0.2) (layer "B.Cu") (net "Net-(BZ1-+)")))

